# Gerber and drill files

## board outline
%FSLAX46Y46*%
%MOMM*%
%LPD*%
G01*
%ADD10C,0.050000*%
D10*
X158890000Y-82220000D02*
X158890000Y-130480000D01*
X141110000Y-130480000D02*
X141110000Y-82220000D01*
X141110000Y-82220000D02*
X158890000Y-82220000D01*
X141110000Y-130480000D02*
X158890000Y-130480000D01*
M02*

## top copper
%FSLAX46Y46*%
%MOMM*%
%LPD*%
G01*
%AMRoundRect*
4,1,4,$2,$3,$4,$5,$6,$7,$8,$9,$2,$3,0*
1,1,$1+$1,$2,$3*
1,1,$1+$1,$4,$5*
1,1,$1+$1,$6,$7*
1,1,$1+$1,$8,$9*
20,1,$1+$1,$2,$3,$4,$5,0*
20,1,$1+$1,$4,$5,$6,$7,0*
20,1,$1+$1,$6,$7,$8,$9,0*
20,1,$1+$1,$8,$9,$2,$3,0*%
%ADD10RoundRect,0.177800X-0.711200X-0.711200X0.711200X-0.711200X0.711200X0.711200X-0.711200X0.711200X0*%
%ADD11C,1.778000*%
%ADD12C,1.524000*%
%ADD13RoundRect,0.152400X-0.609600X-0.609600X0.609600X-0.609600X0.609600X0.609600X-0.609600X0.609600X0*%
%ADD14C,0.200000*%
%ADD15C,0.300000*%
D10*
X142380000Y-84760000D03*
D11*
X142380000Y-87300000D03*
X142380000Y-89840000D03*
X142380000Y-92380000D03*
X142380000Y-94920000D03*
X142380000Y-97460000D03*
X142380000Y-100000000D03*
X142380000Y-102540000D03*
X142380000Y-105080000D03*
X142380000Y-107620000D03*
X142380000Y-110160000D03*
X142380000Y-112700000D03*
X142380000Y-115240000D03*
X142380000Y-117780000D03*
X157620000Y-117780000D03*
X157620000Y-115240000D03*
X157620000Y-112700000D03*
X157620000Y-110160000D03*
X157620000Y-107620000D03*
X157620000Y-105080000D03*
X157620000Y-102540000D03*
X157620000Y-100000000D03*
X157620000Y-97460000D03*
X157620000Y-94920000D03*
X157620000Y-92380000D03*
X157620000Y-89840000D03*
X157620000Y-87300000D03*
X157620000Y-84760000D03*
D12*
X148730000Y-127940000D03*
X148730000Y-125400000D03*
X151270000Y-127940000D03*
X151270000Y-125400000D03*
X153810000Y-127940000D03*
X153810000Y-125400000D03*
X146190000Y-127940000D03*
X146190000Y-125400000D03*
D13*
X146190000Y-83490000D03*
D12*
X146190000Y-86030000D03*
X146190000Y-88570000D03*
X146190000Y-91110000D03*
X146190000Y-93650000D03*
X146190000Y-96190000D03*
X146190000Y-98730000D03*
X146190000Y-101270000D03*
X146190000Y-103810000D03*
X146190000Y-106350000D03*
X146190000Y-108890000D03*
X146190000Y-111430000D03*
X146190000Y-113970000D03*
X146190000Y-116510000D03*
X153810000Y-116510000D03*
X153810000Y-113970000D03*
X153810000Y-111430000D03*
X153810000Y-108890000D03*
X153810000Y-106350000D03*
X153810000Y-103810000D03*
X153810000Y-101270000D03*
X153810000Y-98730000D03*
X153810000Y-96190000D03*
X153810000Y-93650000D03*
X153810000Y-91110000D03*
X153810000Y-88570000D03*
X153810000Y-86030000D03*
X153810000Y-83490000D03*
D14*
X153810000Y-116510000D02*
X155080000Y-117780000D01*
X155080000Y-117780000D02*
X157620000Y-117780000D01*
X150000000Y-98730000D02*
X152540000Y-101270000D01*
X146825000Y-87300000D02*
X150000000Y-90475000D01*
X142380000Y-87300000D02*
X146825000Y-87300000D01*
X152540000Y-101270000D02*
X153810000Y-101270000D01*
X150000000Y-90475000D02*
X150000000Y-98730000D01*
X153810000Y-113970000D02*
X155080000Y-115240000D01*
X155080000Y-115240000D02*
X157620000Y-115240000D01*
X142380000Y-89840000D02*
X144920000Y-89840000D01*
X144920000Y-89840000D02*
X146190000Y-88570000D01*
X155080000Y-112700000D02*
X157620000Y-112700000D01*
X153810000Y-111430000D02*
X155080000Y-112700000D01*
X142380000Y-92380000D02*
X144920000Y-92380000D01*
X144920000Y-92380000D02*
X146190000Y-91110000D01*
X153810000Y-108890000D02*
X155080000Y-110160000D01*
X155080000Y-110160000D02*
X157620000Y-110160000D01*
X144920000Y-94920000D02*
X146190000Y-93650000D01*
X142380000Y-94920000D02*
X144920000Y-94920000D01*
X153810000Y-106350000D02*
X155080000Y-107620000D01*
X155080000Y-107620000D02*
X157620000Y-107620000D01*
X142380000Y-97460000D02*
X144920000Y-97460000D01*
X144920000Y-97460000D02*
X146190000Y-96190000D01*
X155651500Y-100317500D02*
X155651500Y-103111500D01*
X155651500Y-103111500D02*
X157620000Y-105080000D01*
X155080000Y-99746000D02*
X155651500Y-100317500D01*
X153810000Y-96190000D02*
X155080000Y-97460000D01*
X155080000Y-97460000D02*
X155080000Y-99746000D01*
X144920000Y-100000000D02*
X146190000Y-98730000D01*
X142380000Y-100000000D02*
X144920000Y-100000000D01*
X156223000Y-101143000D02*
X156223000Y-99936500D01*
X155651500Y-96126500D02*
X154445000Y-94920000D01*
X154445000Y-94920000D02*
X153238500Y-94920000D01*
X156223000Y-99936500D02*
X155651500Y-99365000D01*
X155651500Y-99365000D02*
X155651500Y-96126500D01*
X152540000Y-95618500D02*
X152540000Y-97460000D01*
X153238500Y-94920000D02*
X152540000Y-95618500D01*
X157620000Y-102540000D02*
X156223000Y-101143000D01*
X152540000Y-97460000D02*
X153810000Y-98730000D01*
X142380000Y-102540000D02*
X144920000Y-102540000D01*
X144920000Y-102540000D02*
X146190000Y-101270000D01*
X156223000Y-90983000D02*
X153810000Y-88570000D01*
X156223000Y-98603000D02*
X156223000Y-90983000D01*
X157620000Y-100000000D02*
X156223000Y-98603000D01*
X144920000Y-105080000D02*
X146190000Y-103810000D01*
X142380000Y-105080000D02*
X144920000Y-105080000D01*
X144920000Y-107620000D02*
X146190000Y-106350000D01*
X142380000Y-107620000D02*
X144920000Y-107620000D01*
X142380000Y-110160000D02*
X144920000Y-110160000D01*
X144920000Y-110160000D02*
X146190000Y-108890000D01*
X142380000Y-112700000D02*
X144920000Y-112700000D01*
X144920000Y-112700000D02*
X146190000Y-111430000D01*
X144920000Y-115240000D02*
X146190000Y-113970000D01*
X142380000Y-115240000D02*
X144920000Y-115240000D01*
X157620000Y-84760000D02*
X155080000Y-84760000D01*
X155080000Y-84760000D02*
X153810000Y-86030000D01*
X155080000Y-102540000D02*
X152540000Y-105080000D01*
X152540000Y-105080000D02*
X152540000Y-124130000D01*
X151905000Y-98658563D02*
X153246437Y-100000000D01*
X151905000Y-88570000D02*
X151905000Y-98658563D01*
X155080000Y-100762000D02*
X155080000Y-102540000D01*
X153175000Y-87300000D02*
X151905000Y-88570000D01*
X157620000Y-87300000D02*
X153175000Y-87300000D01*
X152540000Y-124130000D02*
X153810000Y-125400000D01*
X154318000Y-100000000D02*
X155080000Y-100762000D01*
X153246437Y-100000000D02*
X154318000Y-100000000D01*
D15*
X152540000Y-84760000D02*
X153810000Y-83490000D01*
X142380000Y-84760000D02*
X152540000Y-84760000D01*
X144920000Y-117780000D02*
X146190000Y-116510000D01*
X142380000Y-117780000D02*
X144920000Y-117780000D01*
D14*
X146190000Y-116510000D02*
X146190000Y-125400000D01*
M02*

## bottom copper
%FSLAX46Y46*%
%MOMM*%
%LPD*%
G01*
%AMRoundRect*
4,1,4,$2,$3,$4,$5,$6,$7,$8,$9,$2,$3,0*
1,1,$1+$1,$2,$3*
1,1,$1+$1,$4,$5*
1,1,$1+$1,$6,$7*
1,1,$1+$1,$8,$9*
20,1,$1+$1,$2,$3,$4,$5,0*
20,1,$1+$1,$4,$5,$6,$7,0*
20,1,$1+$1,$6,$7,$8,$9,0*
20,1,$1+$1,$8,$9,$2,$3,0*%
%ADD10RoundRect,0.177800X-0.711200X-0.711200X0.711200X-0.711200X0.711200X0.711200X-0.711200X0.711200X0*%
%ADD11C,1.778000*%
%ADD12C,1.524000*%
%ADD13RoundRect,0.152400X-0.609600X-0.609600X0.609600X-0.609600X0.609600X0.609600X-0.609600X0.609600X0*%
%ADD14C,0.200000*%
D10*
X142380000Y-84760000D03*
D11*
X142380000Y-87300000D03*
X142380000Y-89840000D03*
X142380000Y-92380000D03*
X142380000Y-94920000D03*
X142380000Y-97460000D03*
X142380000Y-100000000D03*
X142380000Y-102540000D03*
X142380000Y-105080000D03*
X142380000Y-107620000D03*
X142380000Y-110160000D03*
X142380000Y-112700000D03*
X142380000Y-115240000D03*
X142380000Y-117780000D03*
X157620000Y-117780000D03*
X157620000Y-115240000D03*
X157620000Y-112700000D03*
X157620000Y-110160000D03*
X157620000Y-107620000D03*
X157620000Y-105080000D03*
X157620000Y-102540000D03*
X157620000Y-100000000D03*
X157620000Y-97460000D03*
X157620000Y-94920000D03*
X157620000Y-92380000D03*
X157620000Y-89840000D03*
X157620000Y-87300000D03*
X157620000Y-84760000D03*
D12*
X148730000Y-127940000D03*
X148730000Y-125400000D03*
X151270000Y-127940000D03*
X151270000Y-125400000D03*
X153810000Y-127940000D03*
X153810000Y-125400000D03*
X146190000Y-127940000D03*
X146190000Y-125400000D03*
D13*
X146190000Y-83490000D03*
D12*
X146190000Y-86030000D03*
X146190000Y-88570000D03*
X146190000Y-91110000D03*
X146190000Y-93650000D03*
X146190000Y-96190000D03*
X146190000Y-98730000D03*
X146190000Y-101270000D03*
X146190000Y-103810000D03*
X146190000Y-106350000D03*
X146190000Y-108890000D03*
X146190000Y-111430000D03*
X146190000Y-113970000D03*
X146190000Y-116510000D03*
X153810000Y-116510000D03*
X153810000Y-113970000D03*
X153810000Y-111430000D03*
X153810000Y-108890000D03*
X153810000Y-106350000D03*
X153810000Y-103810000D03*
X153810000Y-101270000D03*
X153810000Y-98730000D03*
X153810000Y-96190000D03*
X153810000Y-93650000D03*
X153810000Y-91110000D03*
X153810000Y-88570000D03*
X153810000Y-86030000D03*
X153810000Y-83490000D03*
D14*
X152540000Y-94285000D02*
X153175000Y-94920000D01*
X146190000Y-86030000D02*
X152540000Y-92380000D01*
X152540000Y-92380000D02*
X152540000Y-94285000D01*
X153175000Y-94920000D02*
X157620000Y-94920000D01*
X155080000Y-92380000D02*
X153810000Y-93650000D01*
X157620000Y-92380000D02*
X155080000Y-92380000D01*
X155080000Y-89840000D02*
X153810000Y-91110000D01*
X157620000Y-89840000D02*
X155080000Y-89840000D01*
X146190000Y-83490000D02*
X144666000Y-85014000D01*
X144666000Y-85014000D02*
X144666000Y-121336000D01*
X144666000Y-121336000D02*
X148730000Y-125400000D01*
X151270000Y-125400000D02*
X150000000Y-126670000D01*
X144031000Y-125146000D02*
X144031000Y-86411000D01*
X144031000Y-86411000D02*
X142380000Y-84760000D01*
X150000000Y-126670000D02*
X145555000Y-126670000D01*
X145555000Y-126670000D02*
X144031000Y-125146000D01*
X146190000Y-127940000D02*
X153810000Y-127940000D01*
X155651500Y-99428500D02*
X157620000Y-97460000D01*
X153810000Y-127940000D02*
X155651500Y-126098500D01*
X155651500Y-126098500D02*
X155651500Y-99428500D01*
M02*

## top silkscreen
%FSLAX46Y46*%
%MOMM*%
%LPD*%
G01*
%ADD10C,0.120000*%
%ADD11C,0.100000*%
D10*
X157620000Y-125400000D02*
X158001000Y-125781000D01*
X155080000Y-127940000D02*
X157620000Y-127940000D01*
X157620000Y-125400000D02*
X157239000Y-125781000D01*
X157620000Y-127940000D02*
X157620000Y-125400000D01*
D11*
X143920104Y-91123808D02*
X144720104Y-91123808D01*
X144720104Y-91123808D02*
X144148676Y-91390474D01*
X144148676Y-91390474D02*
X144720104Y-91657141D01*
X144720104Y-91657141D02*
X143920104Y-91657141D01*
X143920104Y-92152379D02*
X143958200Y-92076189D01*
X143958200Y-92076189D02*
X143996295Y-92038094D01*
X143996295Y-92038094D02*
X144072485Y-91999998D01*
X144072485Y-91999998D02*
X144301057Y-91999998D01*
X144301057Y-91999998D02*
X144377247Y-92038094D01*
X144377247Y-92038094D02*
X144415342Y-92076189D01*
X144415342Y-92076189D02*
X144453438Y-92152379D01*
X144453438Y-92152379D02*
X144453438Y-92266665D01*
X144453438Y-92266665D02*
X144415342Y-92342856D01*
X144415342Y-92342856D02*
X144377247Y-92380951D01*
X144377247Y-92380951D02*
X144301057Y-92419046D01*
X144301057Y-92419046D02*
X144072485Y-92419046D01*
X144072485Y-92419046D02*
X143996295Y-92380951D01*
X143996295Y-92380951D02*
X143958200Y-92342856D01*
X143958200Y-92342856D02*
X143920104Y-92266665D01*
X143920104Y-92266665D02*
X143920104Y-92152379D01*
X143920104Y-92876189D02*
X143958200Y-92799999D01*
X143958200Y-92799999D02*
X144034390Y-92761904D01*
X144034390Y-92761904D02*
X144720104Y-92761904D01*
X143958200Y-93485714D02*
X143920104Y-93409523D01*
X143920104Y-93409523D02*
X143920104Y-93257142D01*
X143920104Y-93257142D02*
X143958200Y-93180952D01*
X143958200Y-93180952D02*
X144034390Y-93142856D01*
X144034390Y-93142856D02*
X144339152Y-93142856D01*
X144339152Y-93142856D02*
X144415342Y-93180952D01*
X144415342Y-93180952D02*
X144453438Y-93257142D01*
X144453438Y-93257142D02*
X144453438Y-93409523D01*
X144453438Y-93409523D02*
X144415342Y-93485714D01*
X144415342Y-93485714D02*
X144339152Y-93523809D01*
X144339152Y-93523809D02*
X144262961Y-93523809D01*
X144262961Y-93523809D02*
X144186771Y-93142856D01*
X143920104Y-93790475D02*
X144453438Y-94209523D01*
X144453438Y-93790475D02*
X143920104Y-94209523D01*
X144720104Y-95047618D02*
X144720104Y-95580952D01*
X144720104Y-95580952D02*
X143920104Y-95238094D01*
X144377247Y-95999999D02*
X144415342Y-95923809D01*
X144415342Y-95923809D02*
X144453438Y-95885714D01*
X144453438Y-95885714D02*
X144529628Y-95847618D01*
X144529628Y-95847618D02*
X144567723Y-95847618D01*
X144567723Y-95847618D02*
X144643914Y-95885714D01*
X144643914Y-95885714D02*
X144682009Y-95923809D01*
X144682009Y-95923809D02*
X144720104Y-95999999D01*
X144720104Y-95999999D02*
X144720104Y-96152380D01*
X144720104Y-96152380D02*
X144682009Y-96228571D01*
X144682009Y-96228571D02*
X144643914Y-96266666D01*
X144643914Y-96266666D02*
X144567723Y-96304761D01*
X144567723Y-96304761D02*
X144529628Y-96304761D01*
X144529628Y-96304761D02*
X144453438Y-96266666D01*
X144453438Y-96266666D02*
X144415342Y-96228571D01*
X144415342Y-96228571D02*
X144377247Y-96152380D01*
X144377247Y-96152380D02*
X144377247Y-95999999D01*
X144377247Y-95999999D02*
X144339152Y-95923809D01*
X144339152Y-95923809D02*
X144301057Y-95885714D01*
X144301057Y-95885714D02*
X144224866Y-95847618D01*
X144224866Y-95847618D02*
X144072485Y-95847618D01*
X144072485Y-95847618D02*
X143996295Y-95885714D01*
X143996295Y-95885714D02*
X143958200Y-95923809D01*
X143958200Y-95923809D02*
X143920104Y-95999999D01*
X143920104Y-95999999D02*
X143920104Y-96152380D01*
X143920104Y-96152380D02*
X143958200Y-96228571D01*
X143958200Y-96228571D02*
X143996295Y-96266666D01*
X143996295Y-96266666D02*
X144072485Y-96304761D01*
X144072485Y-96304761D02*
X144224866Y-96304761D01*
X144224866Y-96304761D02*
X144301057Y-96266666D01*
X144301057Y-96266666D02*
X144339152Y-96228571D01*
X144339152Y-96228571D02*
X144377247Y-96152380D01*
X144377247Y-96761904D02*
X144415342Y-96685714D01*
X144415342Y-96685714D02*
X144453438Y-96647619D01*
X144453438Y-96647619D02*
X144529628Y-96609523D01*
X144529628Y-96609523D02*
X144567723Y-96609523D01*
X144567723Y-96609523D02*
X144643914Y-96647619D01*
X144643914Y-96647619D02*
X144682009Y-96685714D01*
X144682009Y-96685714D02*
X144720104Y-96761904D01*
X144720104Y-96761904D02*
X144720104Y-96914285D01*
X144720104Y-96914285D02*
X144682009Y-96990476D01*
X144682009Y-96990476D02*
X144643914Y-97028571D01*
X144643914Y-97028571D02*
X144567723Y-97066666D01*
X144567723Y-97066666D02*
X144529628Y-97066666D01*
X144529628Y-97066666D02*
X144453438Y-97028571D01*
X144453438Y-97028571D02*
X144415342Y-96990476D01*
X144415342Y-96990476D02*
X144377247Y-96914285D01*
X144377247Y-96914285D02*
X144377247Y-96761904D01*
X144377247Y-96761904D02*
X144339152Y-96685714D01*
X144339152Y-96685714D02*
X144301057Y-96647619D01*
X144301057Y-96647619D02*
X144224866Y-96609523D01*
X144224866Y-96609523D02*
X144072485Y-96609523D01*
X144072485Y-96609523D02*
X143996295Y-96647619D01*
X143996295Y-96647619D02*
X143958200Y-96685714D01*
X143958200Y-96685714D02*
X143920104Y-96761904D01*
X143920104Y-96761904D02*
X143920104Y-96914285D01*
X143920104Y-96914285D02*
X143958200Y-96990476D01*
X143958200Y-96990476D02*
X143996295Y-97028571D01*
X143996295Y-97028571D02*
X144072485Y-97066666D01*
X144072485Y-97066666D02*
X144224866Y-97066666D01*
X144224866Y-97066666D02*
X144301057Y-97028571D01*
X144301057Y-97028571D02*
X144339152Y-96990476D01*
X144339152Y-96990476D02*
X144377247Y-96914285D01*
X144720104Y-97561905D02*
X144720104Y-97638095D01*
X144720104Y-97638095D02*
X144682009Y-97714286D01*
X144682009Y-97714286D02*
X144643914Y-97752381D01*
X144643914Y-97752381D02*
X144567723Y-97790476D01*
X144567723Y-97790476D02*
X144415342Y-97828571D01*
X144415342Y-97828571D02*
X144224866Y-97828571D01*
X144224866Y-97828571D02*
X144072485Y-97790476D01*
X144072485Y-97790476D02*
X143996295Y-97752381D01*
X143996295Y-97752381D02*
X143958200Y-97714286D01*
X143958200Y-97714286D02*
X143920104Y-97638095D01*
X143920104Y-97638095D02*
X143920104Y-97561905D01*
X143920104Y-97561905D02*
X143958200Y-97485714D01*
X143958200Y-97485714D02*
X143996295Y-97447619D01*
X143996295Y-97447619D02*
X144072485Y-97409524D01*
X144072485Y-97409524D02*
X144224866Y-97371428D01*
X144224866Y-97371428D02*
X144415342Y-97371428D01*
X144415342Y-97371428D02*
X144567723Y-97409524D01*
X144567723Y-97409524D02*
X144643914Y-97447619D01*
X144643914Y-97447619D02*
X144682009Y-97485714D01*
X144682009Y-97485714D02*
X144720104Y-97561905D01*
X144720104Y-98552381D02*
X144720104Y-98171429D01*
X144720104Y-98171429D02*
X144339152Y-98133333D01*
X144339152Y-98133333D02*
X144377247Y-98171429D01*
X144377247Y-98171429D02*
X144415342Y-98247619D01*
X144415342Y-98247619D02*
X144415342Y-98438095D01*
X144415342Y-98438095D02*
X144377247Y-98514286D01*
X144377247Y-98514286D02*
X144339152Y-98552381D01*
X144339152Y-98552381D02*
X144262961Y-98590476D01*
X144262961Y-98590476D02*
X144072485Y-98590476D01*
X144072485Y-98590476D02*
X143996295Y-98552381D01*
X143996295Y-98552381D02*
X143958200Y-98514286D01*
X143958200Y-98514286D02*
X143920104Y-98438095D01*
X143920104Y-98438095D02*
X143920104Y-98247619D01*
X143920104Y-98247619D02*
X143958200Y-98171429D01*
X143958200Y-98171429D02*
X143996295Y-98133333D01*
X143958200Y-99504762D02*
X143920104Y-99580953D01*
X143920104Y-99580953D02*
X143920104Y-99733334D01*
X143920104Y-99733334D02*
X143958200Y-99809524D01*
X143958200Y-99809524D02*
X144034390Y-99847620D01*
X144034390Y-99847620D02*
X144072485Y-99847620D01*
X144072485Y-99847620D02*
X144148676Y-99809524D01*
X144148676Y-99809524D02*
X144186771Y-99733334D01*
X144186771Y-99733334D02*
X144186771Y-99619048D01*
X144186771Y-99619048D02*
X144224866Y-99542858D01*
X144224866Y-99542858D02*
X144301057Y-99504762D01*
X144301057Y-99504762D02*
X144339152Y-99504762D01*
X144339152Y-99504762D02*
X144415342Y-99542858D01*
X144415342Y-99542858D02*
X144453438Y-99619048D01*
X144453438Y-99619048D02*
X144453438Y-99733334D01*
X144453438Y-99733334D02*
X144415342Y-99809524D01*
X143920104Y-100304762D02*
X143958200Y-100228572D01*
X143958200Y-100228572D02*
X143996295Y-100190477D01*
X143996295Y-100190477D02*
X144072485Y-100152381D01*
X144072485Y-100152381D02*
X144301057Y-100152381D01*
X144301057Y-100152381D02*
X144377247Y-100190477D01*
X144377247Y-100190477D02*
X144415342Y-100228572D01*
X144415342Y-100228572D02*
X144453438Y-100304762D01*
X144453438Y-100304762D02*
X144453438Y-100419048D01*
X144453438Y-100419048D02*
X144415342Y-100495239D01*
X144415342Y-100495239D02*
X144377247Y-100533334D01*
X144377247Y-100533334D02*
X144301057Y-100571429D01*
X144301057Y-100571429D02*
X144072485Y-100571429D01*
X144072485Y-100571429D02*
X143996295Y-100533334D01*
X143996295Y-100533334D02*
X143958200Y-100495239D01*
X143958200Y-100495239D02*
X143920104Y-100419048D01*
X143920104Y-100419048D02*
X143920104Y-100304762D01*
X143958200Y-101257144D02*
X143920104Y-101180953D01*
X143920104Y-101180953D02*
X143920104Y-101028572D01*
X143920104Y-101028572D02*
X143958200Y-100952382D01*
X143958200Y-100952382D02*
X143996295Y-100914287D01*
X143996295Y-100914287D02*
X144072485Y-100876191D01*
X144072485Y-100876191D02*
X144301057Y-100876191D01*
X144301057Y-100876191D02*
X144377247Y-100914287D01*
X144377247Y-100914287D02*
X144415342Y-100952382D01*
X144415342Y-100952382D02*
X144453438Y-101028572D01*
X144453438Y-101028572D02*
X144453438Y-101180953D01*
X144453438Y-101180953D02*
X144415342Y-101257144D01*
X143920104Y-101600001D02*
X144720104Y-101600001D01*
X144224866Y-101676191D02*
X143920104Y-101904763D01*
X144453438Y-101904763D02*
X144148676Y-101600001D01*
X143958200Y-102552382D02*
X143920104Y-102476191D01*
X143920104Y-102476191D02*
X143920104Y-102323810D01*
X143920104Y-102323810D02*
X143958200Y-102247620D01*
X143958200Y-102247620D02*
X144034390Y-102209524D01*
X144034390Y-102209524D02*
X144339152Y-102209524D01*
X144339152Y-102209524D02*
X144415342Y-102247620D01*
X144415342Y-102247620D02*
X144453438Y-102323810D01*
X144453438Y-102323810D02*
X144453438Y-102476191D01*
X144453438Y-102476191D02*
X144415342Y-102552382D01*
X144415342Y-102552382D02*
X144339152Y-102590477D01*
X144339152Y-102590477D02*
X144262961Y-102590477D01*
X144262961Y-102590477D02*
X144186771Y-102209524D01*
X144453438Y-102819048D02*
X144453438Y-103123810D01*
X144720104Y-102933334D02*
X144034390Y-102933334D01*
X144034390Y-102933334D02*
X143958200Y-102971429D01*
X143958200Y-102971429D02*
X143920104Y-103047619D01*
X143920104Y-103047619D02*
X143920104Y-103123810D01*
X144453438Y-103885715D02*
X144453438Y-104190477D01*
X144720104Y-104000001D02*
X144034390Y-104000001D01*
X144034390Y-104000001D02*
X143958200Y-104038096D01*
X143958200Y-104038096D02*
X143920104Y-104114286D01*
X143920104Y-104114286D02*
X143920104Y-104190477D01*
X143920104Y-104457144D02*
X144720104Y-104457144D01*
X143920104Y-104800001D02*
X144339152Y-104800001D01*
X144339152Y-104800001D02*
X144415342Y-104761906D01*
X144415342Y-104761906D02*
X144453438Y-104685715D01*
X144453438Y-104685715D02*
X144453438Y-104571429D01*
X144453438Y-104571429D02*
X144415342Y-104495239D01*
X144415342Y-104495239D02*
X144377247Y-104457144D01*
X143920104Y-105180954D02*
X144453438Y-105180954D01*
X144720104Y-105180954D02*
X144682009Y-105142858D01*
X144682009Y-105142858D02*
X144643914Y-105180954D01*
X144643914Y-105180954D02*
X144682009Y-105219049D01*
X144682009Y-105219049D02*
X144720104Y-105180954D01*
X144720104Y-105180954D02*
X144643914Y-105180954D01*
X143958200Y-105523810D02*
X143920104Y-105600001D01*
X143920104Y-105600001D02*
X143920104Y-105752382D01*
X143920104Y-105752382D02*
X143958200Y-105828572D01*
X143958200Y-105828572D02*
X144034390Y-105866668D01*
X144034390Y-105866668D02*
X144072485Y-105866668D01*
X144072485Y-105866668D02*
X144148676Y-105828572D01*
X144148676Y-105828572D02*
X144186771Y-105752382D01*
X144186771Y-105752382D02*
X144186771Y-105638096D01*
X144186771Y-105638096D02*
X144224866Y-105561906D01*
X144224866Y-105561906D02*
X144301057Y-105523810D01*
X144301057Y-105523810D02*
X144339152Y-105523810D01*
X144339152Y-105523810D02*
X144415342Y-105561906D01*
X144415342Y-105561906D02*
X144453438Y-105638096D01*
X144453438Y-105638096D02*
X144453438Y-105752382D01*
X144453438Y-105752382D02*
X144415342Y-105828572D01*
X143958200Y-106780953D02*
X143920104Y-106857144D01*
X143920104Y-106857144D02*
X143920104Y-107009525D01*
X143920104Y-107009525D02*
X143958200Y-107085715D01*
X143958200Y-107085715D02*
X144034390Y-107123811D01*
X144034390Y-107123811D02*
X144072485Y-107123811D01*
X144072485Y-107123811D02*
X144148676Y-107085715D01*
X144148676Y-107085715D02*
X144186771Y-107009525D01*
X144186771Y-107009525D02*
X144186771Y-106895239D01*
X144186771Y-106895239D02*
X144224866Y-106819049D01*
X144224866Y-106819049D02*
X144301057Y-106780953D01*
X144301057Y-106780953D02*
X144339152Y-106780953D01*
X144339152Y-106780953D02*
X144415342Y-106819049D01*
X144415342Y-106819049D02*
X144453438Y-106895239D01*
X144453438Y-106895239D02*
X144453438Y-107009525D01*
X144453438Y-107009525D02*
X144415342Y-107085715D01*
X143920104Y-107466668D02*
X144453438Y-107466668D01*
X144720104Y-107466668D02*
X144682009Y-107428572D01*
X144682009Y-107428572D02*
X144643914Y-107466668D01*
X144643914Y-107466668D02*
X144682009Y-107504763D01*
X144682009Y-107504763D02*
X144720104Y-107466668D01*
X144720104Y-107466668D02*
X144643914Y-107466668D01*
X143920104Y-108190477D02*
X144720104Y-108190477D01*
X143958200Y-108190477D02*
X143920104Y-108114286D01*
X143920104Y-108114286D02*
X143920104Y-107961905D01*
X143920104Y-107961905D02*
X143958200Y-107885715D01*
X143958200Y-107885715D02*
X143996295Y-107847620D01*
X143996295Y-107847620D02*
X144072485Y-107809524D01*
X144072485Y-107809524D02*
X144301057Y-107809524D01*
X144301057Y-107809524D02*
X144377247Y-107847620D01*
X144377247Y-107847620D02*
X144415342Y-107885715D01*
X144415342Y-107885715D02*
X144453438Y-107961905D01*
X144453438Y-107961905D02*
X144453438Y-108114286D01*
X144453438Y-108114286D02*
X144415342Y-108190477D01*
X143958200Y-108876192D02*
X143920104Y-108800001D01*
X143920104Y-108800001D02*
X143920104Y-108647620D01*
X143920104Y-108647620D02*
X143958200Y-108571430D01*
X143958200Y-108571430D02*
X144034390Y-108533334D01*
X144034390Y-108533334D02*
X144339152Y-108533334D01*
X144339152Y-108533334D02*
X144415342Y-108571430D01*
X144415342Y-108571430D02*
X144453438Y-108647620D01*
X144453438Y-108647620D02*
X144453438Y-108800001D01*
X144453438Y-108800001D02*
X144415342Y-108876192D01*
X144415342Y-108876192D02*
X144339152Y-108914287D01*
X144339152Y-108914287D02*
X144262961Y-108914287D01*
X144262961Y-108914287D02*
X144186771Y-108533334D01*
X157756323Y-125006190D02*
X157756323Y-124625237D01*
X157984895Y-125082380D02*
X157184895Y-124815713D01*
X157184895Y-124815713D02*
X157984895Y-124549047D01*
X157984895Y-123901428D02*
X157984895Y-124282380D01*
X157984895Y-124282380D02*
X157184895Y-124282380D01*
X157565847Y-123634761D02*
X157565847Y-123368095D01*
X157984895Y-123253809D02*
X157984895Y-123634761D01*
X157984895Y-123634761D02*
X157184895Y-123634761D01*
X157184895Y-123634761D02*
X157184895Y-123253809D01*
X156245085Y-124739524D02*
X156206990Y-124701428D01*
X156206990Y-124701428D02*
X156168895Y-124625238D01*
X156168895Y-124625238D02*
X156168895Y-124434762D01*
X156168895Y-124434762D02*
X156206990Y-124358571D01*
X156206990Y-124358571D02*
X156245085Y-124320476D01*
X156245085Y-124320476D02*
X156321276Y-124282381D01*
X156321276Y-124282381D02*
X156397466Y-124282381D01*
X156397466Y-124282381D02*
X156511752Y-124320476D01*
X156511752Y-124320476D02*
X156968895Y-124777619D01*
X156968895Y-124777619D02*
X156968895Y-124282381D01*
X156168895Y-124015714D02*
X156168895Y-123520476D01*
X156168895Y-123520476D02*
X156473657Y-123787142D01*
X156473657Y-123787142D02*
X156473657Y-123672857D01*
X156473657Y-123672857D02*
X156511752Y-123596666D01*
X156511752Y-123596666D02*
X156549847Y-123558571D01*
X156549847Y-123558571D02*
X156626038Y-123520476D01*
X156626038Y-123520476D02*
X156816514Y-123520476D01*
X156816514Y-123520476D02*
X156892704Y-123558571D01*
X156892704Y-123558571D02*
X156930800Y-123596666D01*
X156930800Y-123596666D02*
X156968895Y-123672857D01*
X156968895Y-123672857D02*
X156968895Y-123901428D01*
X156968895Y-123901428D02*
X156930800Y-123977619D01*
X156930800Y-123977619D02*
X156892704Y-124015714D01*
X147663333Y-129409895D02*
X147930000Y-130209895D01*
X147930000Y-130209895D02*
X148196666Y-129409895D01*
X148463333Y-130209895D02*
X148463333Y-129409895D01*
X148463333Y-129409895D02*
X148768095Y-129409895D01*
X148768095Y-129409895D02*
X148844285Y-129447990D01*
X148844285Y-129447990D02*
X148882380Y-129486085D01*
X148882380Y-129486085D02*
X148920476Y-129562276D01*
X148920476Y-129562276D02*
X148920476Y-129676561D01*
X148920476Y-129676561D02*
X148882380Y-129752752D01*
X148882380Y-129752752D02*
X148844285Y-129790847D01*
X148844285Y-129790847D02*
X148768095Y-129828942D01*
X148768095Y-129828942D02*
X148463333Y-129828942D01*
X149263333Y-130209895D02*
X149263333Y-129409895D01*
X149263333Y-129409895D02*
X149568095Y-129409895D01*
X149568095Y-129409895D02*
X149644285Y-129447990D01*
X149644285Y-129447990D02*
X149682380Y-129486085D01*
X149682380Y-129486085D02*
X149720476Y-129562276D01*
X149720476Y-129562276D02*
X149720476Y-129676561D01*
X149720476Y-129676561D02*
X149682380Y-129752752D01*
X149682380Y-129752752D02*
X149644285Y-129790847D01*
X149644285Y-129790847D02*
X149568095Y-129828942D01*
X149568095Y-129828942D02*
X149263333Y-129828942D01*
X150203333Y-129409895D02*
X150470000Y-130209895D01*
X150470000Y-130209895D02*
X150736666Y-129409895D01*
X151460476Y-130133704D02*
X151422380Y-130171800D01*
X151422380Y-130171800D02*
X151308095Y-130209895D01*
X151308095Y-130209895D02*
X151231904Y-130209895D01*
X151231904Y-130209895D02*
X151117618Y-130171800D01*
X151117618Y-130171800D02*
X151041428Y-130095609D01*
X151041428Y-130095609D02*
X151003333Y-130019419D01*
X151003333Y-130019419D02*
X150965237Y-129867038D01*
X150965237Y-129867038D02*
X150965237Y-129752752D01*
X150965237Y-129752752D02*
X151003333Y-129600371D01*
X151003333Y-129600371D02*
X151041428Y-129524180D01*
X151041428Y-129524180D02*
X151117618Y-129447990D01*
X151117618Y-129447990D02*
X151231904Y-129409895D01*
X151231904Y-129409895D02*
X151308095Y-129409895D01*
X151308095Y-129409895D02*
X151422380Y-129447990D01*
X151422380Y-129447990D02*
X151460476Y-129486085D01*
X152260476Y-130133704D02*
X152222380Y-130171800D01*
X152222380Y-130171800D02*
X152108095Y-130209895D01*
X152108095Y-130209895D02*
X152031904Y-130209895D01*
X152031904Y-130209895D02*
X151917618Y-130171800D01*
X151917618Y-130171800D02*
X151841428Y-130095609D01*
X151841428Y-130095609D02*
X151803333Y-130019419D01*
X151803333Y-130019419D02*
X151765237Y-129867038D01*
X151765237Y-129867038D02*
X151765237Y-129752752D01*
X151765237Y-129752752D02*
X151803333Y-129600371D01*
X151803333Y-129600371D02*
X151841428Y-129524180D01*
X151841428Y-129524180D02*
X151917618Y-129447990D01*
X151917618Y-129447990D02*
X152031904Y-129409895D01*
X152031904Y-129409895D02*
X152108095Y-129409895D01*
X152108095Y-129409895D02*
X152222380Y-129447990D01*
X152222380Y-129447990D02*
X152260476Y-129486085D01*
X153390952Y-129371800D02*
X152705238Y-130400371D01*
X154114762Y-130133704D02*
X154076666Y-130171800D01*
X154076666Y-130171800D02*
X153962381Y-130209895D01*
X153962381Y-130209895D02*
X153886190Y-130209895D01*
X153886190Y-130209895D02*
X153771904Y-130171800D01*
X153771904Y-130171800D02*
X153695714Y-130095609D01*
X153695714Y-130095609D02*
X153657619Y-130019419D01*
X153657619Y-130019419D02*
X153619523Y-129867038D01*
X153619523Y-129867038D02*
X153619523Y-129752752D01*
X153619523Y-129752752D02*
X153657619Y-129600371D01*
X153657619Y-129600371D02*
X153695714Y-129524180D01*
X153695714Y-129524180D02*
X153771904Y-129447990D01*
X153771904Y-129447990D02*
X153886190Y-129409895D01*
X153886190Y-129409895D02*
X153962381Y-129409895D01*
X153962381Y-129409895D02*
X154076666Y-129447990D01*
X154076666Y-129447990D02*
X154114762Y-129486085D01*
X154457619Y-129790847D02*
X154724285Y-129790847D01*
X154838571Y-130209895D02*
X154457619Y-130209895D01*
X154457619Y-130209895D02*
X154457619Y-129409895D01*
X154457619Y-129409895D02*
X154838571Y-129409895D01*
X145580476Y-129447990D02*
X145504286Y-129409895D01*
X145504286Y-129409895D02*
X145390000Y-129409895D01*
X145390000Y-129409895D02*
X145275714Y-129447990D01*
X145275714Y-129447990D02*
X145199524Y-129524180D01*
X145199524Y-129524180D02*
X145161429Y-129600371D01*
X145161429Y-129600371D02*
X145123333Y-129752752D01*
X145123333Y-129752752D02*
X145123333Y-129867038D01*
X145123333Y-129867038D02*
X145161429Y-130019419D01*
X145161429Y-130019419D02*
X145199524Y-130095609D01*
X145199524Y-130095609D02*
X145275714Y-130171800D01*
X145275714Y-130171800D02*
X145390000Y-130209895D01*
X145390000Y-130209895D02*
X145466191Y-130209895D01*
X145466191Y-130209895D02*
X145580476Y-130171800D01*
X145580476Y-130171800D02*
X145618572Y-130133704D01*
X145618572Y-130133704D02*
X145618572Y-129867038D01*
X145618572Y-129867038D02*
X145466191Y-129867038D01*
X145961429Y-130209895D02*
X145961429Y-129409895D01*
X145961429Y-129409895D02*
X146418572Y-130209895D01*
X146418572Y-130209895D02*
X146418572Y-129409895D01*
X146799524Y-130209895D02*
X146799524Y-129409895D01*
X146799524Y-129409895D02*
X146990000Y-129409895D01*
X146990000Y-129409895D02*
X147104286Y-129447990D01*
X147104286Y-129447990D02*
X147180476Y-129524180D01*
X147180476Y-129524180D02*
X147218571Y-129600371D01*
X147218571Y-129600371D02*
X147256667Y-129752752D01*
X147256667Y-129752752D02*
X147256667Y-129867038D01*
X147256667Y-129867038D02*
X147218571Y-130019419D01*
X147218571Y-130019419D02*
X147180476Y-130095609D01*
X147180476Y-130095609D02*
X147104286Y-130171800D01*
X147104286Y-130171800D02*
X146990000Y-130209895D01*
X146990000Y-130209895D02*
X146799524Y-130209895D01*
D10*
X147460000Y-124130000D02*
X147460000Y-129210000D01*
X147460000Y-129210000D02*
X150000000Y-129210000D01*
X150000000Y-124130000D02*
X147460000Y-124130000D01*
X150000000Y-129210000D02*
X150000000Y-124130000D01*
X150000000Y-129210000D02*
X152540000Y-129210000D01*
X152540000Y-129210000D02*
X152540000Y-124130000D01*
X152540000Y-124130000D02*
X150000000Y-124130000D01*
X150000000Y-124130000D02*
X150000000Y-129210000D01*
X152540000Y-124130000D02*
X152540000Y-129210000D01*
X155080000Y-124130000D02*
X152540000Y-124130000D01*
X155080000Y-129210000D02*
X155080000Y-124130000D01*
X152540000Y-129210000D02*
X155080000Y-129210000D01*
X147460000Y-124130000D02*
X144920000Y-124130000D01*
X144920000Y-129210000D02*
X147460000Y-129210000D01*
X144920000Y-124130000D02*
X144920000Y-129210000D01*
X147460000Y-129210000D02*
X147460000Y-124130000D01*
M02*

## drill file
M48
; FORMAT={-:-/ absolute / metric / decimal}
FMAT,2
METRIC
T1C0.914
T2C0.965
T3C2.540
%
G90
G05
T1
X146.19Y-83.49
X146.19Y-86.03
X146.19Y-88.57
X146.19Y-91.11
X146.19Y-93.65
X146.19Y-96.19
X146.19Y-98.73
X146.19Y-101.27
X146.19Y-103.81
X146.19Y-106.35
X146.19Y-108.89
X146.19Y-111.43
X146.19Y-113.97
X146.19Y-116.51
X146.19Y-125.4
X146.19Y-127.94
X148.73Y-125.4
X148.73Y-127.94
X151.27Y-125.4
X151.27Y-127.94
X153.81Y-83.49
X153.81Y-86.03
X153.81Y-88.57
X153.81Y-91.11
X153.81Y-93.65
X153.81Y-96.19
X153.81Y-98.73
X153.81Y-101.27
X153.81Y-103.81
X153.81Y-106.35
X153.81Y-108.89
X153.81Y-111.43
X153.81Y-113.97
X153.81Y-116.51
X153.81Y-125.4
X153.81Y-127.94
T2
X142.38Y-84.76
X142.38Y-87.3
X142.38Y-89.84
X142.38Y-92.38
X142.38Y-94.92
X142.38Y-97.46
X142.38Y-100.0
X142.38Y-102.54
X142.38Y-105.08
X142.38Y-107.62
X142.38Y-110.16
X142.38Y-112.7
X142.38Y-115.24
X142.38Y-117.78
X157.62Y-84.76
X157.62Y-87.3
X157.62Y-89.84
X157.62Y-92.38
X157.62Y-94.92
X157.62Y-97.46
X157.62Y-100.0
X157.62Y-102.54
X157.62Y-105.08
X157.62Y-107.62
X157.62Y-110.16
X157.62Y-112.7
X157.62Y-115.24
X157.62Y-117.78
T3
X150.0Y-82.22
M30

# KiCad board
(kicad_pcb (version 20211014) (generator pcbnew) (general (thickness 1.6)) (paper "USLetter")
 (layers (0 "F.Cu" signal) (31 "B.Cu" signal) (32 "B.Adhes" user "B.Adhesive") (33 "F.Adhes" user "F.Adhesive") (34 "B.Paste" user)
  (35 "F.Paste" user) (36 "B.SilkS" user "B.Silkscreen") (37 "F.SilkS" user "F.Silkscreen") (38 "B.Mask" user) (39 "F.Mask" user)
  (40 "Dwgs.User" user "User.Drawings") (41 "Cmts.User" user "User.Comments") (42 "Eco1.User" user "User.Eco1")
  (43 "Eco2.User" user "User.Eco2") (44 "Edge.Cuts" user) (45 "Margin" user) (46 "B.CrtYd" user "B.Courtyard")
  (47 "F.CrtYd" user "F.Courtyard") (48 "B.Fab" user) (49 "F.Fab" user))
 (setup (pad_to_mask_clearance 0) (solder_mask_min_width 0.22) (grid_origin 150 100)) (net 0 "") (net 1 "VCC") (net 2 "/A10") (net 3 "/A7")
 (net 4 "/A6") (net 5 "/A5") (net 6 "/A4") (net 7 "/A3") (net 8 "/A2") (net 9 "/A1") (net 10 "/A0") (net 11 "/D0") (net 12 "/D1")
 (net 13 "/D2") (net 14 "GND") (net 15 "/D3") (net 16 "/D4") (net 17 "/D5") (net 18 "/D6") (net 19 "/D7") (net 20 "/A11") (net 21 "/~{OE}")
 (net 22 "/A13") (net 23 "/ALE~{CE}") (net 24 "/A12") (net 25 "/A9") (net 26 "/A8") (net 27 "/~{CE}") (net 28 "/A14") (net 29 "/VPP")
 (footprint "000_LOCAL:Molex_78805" (layer "F.Cu") (at 150 101.27)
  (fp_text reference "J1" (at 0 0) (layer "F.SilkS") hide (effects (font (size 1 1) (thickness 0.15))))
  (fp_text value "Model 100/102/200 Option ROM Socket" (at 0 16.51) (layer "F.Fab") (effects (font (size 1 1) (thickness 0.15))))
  (pad "1" thru_hole roundrect locked (at -7.62 -16.51) (size 1.778 1.778) (drill 0.9652) (layers *.Cu *.Mask) (roundrect_rratio 0.1)
   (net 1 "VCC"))
  (pad "2" thru_hole circle locked (at -7.62 -13.97) (size 1.778 1.778) (drill 0.9652) (layers *.Cu *.Mask) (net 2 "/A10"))
  (pad "3" thru_hole circle locked (at -7.62 -11.43) (size 1.778 1.778) (drill 0.9652) (layers *.Cu *.Mask) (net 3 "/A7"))
  (pad "4" thru_hole circle locked (at -7.62 -8.89) (size 1.778 1.778) (drill 0.9652) (layers *.Cu *.Mask) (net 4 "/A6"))
  (pad "5" thru_hole circle locked (at -7.62 -6.35) (size 1.778 1.778) (drill 0.9652) (layers *.Cu *.Mask) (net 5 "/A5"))
  (pad "6" thru_hole circle locked (at -7.62 -3.81) (size 1.778 1.778) (drill 0.9652) (layers *.Cu *.Mask) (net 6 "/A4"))
  (pad "7" thru_hole circle locked (at -7.62 -1.27) (size 1.778 1.778) (drill 0.9652) (layers *.Cu *.Mask) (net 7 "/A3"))
  (pad "8" thru_hole circle locked (at -7.62 1.27) (size 1.778 1.778) (drill 0.9652) (layers *.Cu *.Mask) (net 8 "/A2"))
  (pad "9" thru_hole circle locked (at -7.62 3.81) (size 1.778 1.778) (drill 0.9652) (layers *.Cu *.Mask) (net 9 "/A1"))
  (pad "10" thru_hole circle locked (at -7.62 6.35) (size 1.778 1.778) (drill 0.9652) (layers *.Cu *.Mask) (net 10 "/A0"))
  (pad "11" thru_hole circle locked (at -7.62 8.89) (size 1.778 1.778) (drill 0.9652) (layers *.Cu *.Mask) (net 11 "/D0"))
  (pad "12" thru_hole circle locked (at -7.62 11.43) (size 1.778 1.778) (drill 0.9652) (layers *.Cu *.Mask) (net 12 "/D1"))
  (pad "13" thru_hole circle locked (at -7.62 13.97) (size 1.778 1.778) (drill 0.9652) (layers *.Cu *.Mask) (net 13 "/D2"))
  (pad "14" thru_hole circle locked (at -7.62 16.51) (size 1.778 1.778) (drill 0.9652) (layers *.Cu *.Mask) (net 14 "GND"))
  (pad "15" thru_hole circle locked (at 7.62 16.51) (size 1.778 1.778) (drill 0.9652) (layers *.Cu *.Mask) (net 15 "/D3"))
  (pad "16" thru_hole circle locked (at 7.62 13.97) (size 1.778 1.778) (drill 0.9652) (layers *.Cu *.Mask) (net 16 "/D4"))
  (pad "17" thru_hole circle locked (at 7.62 11.43) (size 1.778 1.778) (drill 0.9652) (layers *.Cu *.Mask) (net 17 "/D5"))
  (pad "18" thru_hole circle locked (at 7.62 8.89) (size 1.778 1.778) (drill 0.9652) (layers *.Cu *.Mask) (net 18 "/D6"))
  (pad "19" thru_hole circle locked (at 7.62 6.35) (size 1.778 1.778) (drill 0.9652) (layers *.Cu *.Mask) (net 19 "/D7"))
  (pad "20" thru_hole circle locked (at 7.62 3.81) (size 1.778 1.778) (drill 0.9652) (layers *.Cu *.Mask) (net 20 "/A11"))
  (pad "21" thru_hole circle locked (at 7.62 1.27) (size 1.778 1.778) (drill 0.9652) (layers *.Cu *.Mask) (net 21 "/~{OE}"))
  (pad "22" thru_hole circle locked (at 7.62 -1.27) (size 1.778 1.778) (drill 0.9652) (layers *.Cu *.Mask) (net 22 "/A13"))
  (pad "23" thru_hole circle locked (at 7.62 -3.81) (size 1.778 1.778) (drill 0.9652) (layers *.Cu *.Mask) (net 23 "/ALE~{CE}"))
  (pad "24" thru_hole circle locked (at 7.62 -6.35) (size 1.778 1.778) (drill 0.9652) (layers *.Cu *.Mask) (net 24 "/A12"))
  (pad "25" thru_hole circle locked (at 7.62 -8.89) (size 1.778 1.778) (drill 0.9652) (layers *.Cu *.Mask) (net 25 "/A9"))
  (pad "26" thru_hole circle locked (at 7.62 -11.43) (size 1.778 1.778) (drill 0.9652) (layers *.Cu *.Mask) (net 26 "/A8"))
  (pad "27" thru_hole circle locked (at 7.62 -13.97) (size 1.778 1.778) (drill 0.9652) (layers *.Cu *.Mask) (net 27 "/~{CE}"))
  (pad "28" thru_hole circle locked (at 7.62 -16.51) (size 1.778 1.778) (drill 0.9652) (layers *.Cu *.Mask) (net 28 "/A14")))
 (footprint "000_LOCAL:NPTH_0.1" (layer "F.Cu") (at 150 82.22)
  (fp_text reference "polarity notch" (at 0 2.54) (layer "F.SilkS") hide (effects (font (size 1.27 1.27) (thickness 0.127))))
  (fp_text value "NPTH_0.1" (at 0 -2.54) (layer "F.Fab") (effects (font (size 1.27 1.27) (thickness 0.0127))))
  (pad "" np_thru_hole circle locked (at 0 0) (size 2.54 2.54) (drill 2.54) (layers *.Cu *.Mask)))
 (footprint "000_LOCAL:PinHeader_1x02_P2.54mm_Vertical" (layer "F.Cu") (at 148.73 127.94 180)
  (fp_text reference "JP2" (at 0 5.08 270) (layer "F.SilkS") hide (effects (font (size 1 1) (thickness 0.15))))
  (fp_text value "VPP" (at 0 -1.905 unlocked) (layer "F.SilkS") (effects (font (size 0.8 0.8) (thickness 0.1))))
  (fp_line (start 1.27 3.81) (end 1.27 -1.27) (layer "F.SilkS") (width 0.12))
  (fp_line (start 1.27 -1.27) (end -1.27 -1.27) (layer "F.SilkS") (width 0.12))
  (fp_line (start -1.27 3.81) (end 1.27 3.81) (layer "F.SilkS") (width 0.12))
  (fp_line (start -1.27 -1.27) (end -1.27 3.81) (layer "F.SilkS") (width 0.12))
  (pad "1" thru_hole circle locked (at 0 0 180) (size 1.524 1.524) (drill 0.9144) (layers *.Cu *.Mask) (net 23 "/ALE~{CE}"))
  (pad "2" thru_hole circle locked (at 0 2.54 180) (size 1.524 1.524) (drill 0.9144) (layers *.Cu *.Mask) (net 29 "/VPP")))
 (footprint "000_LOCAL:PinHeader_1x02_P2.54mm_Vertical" (layer "F.Cu") (at 151.27 127.94 180)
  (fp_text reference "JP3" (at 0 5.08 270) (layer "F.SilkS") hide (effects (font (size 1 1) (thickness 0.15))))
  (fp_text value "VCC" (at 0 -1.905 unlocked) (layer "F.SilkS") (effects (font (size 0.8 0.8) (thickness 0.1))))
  (fp_line (start 1.27 -1.27) (end -1.27 -1.27) (layer "F.SilkS") (width 0.12))
  (fp_line (start -1.27 -1.27) (end -1.27 3.81) (layer "F.SilkS") (width 0.12))
  (fp_line (start -1.27 3.81) (end 1.27 3.81) (layer "F.SilkS") (width 0.12))
  (fp_line (start 1.27 3.81) (end 1.27 -1.27) (layer "F.SilkS") (width 0.12))
  (pad "1" thru_hole circle locked (at 0 0 180) (size 1.524 1.524) (drill 0.9144) (layers *.Cu *.Mask) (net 23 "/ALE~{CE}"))
  (pad "2" thru_hole circle locked (at 0 2.54 180) (size 1.524 1.524) (drill 0.9144) (layers *.Cu *.Mask) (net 1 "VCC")))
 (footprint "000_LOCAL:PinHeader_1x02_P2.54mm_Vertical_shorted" (layer "F.Cu") (at 153.81 127.94 180)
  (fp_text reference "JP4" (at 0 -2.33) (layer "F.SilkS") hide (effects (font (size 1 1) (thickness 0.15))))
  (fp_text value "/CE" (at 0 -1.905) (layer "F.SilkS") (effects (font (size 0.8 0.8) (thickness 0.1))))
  (fp_line (start 1.27 3.81) (end 1.27 -1.27) (layer "F.SilkS") (width 0.12))
  (fp_line (start -1.27 3.81) (end 1.27 3.81) (layer "F.SilkS") (width 0.12))
  (fp_line (start -1.27 -1.27) (end -1.27 3.81) (layer "F.SilkS") (width 0.12))
  (fp_line (start 1.27 -1.27) (end -1.27 -1.27) (layer "F.SilkS") (width 0.12))
  (pad "1" thru_hole circle locked (at 0 0 180) (size 1.524 1.524) (drill 0.9144) (layers *.Cu *.Mask) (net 23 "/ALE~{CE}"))
  (pad "2" thru_hole circle locked (at 0 2.54 180) (size 1.524 1.524) (drill 0.9144) (layers *.Cu *.Mask) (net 27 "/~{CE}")))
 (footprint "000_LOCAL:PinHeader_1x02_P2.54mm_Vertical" (layer "F.Cu") (at 146.19 127.94 180)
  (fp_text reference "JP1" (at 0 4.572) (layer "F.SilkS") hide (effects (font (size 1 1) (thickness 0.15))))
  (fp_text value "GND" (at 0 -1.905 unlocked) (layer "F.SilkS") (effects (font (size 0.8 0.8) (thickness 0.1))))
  (fp_line (start -1.27 3.81) (end 1.27 3.81) (layer "F.SilkS") (width 0.12))
  (fp_line (start 1.27 -1.27) (end -1.27 -1.27) (layer "F.SilkS") (width 0.12))
  (fp_line (start 1.27 3.81) (end 1.27 -1.27) (layer "F.SilkS") (width 0.12))
  (fp_line (start -1.27 -1.27) (end -1.27 3.81) (layer "F.SilkS") (width 0.12))
  (pad "1" thru_hole circle locked (at 0 0 180) (size 1.524 1.524) (drill 0.9144) (layers *.Cu *.Mask) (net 23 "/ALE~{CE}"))
  (pad "2" thru_hole circle locked (at 0 2.54 180) (size 1.524 1.524) (drill 0.9144) (layers *.Cu *.Mask) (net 14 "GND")))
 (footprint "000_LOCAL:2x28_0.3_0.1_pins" (layer "F.Cu") (at 150 100)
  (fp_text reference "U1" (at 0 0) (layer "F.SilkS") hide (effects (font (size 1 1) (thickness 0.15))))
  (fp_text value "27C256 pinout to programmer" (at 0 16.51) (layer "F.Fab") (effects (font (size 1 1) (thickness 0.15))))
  (pad "1" thru_hole roundrect locked (at -3.81 -16.51) (size 1.524 1.524) (drill 0.9144) (layers *.Cu *.Mask) (roundrect_rratio 0.1)
   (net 29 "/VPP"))
  (pad "2" thru_hole circle locked (at -3.81 -13.97) (size 1.524 1.524) (drill 0.9144) (layers *.Cu *.Mask) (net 24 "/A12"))
  (pad "3" thru_hole circle locked (at -3.81 -11.43) (size 1.524 1.524) (drill 0.9144) (layers *.Cu *.Mask) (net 3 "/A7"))
  (pad "4" thru_hole circle locked (at -3.81 -8.89) (size 1.524 1.524) (drill 0.9144) (layers *.Cu *.Mask) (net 4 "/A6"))
  (pad "5" thru_hole circle locked (at -3.81 -6.35) (size 1.524 1.524) (drill 0.9144) (layers *.Cu *.Mask) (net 5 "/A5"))
  (pad "6" thru_hole circle locked (at -3.81 -3.81) (size 1.524 1.524) (drill 0.9144) (layers *.Cu *.Mask) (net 6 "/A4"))
  (pad "7" thru_hole circle locked (at -3.81 -1.27) (size 1.524 1.524) (drill 0.9144) (layers *.Cu *.Mask) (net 7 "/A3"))
  (pad "8" thru_hole circle locked (at -3.81 1.27) (size 1.524 1.524) (drill 0.9144) (layers *.Cu *.Mask) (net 8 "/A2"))
  (pad "9" thru_hole circle locked (at -3.81 3.81) (size 1.524 1.524) (drill 0.9144) (layers *.Cu *.Mask) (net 9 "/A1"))
  (pad "10" thru_hole circle locked (at -3.81 6.35) (size 1.524 1.524) (drill 0.9144) (layers *.Cu *.Mask) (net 10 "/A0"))
  (pad "11" thru_hole circle locked (at -3.81 8.89) (size 1.524 1.524) (drill 0.9144) (layers *.Cu *.Mask) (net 11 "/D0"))
  (pad "12" thru_hole circle locked (at -3.81 11.43) (size 1.524 1.524) (drill 0.9144) (layers *.Cu *.Mask) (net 12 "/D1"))
  (pad "13" thru_hole circle locked (at -3.81 13.97) (size 1.524 1.524) (drill 0.9144) (layers *.Cu *.Mask) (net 13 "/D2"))
  (pad "14" thru_hole circle locked (at -3.81 16.51) (size 1.524 1.524) (drill 0.9144) (layers *.Cu *.Mask) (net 14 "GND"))
  (pad "15" thru_hole circle locked (at 3.81 16.51) (size 1.524 1.524) (drill 0.9144) (layers *.Cu *.Mask) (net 15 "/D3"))
  (pad "16" thru_hole circle locked (at 3.81 13.97) (size 1.524 1.524) (drill 0.9144) (layers *.Cu *.Mask) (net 16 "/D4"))
  (pad "17" thru_hole circle locked (at 3.81 11.43) (size 1.524 1.524) (drill 0.9144) (layers *.Cu *.Mask) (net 17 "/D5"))
  (pad "18" thru_hole circle locked (at 3.81 8.89) (size 1.524 1.524) (drill 0.9144) (layers *.Cu *.Mask) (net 18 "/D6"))
  (pad "19" thru_hole circle locked (at 3.81 6.35) (size 1.524 1.524) (drill 0.9144) (layers *.Cu *.Mask) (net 19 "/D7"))
  (pad "20" thru_hole circle locked (at 3.81 3.81) (size 1.524 1.524) (drill 0.9144) (layers *.Cu *.Mask) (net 27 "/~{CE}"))
  (pad "21" thru_hole circle locked (at 3.81 1.27) (size 1.524 1.524) (drill 0.9144) (layers *.Cu *.Mask) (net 2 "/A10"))
  (pad "22" thru_hole circle locked (at 3.81 -1.27) (size 1.524 1.524) (drill 0.9144) (layers *.Cu *.Mask) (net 21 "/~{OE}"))
  (pad "23" thru_hole circle locked (at 3.81 -3.81) (size 1.524 1.524) (drill 0.9144) (layers *.Cu *.Mask) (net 20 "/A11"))
  (pad "24" thru_hole circle locked (at 3.81 -6.35) (size 1.524 1.524) (drill 0.9144) (layers *.Cu *.Mask) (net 25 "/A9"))
  (pad "25" thru_hole circle locked (at 3.81 -8.89) (size 1.524 1.524) (drill 0.9144) (layers *.Cu *.Mask) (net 26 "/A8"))
  (pad "26" thru_hole circle locked (at 3.81 -11.43) (size 1.524 1.524) (drill 0.9144) (layers *.Cu *.Mask) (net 22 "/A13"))
  (pad "27" thru_hole circle locked (at 3.81 -13.97) (size 1.524 1.524) (drill 0.9144) (layers *.Cu *.Mask) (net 28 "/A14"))
  (pad "28" thru_hole circle locked (at 3.81 -16.51) (size 1.524 1.524) (drill 0.9144) (layers *.Cu *.Mask) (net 1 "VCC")))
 (gr_line (start 157.62 125.4) (end 158.001 125.781) (layer "F.SilkS") (width 0.12))
 (gr_line (start 155.08 127.94) (end 157.62 127.94) (layer "F.SilkS") (width 0.12))
 (gr_line (start 157.62 125.4) (end 157.239 125.781) (layer "F.SilkS") (width 0.12))
 (gr_line (start 157.62 127.94) (end 157.62 125.4) (layer "F.SilkS") (width 0.12))
 (gr_line (start 158.89 82.22) (end 158.89 130.48) (layer "Edge.Cuts") (width 0.05))
 (gr_line (start 141.11 130.48) (end 141.11 82.22) (layer "Edge.Cuts") (width 0.05))
 (gr_line (start 141.11 82.22) (end 158.89 82.22) (layer "Edge.Cuts") (width 0.05))
 (gr_line (start 141.11 130.48) (end 158.89 130.48) (layer "Edge.Cuts") (width 0.05))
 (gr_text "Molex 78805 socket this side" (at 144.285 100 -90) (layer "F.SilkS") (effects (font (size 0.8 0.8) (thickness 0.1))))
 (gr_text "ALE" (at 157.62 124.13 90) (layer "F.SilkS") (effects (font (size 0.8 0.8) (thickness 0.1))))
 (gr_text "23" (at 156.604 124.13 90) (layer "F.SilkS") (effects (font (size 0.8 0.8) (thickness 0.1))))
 (segment (start 153.81 116.51) (end 155.08 117.78) (width 0.2) (layer "F.Cu") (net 15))
 (segment (start 155.08 117.78) (end 157.62 117.78) (width 0.2) (layer "F.Cu") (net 15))
 (segment (start 150 98.73) (end 152.54 101.27) (width 0.2) (layer "F.Cu") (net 2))
 (segment (start 146.825 87.3) (end 150 90.475) (width 0.2) (layer "F.Cu") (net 2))
 (segment (start 142.38 87.3) (end 146.825 87.3) (width 0.2) (layer "F.Cu") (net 2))
 (segment (start 152.54 101.27) (end 153.81 101.27) (width 0.2) (layer "F.Cu") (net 2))
 (segment (start 150 90.475) (end 150 98.73) (width 0.2) (layer "F.Cu") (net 2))
 (segment (start 153.81 113.97) (end 155.08 115.24) (width 0.2) (layer "F.Cu") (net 16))
 (segment (start 155.08 115.24) (end 157.62 115.24) (width 0.2) (layer "F.Cu") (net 16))
 (segment (start 142.38 89.84) (end 144.92 89.84) (width 0.2) (layer "F.Cu") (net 3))
 (segment (start 144.92 89.84) (end 146.19 88.57) (width 0.2) (layer "F.Cu") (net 3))
 (segment (start 155.08 112.7) (end 157.62 112.7) (width 0.2) (layer "F.Cu") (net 17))
 (segment (start 153.81 111.43) (end 155.08 112.7) (width 0.2) (layer "F.Cu") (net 17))
 (segment (start 142.38 92.38) (end 144.92 92.38) (width 0.2) (layer "F.Cu") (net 4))
 (segment (start 144.92 92.38) (end 146.19 91.11) (width 0.2) (layer "F.Cu") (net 4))
 (segment (start 153.81 108.89) (end 155.08 110.16) (width 0.2) (layer "F.Cu") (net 18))
 (segment (start 155.08 110.16) (end 157.62 110.16) (width 0.2) (layer "F.Cu") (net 18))
 (segment (start 144.92 94.92) (end 146.19 93.65) (width 0.2) (layer "F.Cu") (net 5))
 (segment (start 142.38 94.92) (end 144.92 94.92) (width 0.2) (layer "F.Cu") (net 5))
 (segment (start 153.81 106.35) (end 155.08 107.62) (width 0.2) (layer "F.Cu") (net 19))
 (segment (start 155.08 107.62) (end 157.62 107.62) (width 0.2) (layer "F.Cu") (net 19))
 (segment (start 142.38 97.46) (end 144.92 97.46) (width 0.2) (layer "F.Cu") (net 6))
 (segment (start 144.92 97.46) (end 146.19 96.19) (width 0.2) (layer "F.Cu") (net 6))
 (segment (start 155.6515 100.3175) (end 155.6515 103.1115) (width 0.2) (layer "F.Cu") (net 20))
 (segment (start 155.6515 103.1115) (end 157.62 105.08) (width 0.2) (layer "F.Cu") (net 20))
 (segment (start 155.08 99.746) (end 155.6515 100.3175) (width 0.2) (layer "F.Cu") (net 20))
 (segment (start 153.81 96.19) (end 155.08 97.46) (width 0.2) (layer "F.Cu") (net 20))
 (segment (start 155.08 97.46) (end 155.08 99.746) (width 0.2) (layer "F.Cu") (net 20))
 (segment (start 144.92 100) (end 146.19 98.73) (width 0.2) (layer "F.Cu") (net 7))
 (segment (start 142.38 100) (end 144.92 100) (width 0.2) (layer "F.Cu") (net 7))
 (segment (start 156.223 101.143) (end 156.223 99.9365) (width 0.2) (layer "F.Cu") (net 21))
 (segment (start 155.6515 96.1265) (end 154.445 94.92) (width 0.2) (layer "F.Cu") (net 21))
 (segment (start 154.445 94.92) (end 153.2385 94.92) (width 0.2) (layer "F.Cu") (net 21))
 (segment (start 156.223 99.9365) (end 155.6515 99.365) (width 0.2) (layer "F.Cu") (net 21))
 (segment (start 155.6515 99.365) (end 155.6515 96.1265) (width 0.2) (layer "F.Cu") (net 21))
 (segment (start 152.54 95.6185) (end 152.54 97.46) (width 0.2) (layer "F.Cu") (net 21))
 (segment (start 153.2385 94.92) (end 152.54 95.6185) (width 0.2) (layer "F.Cu") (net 21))
 (segment (start 157.62 102.54) (end 156.223 101.143) (width 0.2) (layer "F.Cu") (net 21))
 (segment (start 152.54 97.46) (end 153.81 98.73) (width 0.2) (layer "F.Cu") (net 21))
 (segment (start 142.38 102.54) (end 144.92 102.54) (width 0.2) (layer "F.Cu") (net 8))
 (segment (start 144.92 102.54) (end 146.19 101.27) (width 0.2) (layer "F.Cu") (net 8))
 (segment (start 156.223 90.983) (end 153.81 88.57) (width 0.2) (layer "F.Cu") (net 22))
 (segment (start 156.223 98.603) (end 156.223 90.983) (width 0.2) (layer "F.Cu") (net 22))
 (segment (start 157.62 100) (end 156.223 98.603) (width 0.2) (layer "F.Cu") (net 22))
 (segment (start 144.92 105.08) (end 146.19 103.81) (width 0.2) (layer "F.Cu") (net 9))
 (segment (start 142.38 105.08) (end 144.92 105.08) (width 0.2) (layer "F.Cu") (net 9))
 (segment (start 144.92 107.62) (end 146.19 106.35) (width 0.2) (layer "F.Cu") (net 10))
 (segment (start 142.38 107.62) (end 144.92 107.62) (width 0.2) (layer "F.Cu") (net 10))
 (segment (start 152.54 94.285) (end 153.175 94.92) (width 0.2) (layer "B.Cu") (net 24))
 (segment (start 146.19 86.03) (end 152.54 92.38) (width 0.2) (layer "B.Cu") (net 24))
 (segment (start 152.54 92.38) (end 152.54 94.285) (width 0.2) (layer "B.Cu") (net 24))
 (segment (start 153.175 94.92) (end 157.62 94.92) (width 0.2) (layer "B.Cu") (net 24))
 (segment (start 142.38 110.16) (end 144.92 110.16) (width 0.2) (layer "F.Cu") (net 11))
 (segment (start 144.92 110.16) (end 146.19 108.89) (width 0.2) (layer "F.Cu") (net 11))
 (segment (start 155.08 92.38) (end 153.81 93.65) (width 0.2) (layer "B.Cu") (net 25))
 (segment (start 157.62 92.38) (end 155.08 92.38) (width 0.2) (layer "B.Cu") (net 25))
 (segment (start 142.38 112.7) (end 144.92 112.7) (width 0.2) (layer "F.Cu") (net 12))
 (segment (start 144.92 112.7) (end 146.19 111.43) (width 0.2) (layer "F.Cu") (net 12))
 (segment (start 155.08 89.84) (end 153.81 91.11) (width 0.2) (layer "B.Cu") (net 26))
 (segment (start 157.62 89.84) (end 155.08 89.84) (width 0.2) (layer "B.Cu") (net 26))
 (segment (start 144.92 115.24) (end 146.19 113.97) (width 0.2) (layer "F.Cu") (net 13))
 (segment (start 142.38 115.24) (end 144.92 115.24) (width 0.2) (layer "F.Cu") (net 13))
 (segment (start 157.62 84.76) (end 155.08 84.76) (width 0.2) (layer "F.Cu") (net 28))
 (segment (start 155.08 84.76) (end 153.81 86.03) (width 0.2) (layer "F.Cu") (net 28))
 (segment (start 155.08 102.54) (end 152.54 105.08) (width 0.2) (layer "F.Cu") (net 27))
 (segment (start 152.54 105.08) (end 152.54 124.13) (width 0.2) (layer "F.Cu") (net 27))
 (segment (start 151.905 98.658563) (end 153.246437 100) (width 0.2) (layer "F.Cu") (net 27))
 (segment (start 151.905 88.57) (end 151.905 98.658563) (width 0.2) (layer "F.Cu") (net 27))
 (segment (start 155.08 100.762) (end 155.08 102.54) (width 0.2) (layer "F.Cu") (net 27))
 (segment (start 153.175 87.3) (end 151.905 88.57) (width 0.2) (layer "F.Cu") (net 27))
 (segment (start 157.62 87.3) (end 153.175 87.3) (width 0.2) (layer "F.Cu") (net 27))
 (segment (start 152.54 124.13) (end 153.81 125.4) (width 0.2) (layer "F.Cu") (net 27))
 (segment (start 154.318 100) (end 155.08 100.762) (width 0.2) (layer "F.Cu") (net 27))
 (segment (start 153.246437 100) (end 154.318 100) (width 0.2) (layer "F.Cu") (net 27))
 (segment (start 146.19 83.49) (end 144.666 85.014) (width 0.2) (layer "B.Cu") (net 29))
 (segment (start 144.666 85.014) (end 144.666 121.336) (width 0.2) (layer "B.Cu") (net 29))
 (segment (start 144.666 121.336) (end 148.73 125.4) (width 0.2) (layer "B.Cu") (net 29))
 (segment (start 152.54 84.76) (end 153.81 83.49) (width 0.3) (layer "F.Cu") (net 1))
 (segment (start 142.38 84.76) (end 152.54 84.76) (width 0.3) (layer "F.Cu") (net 1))
 (segment (start 151.27 125.4) (end 150 126.67) (width 0.2) (layer "B.Cu") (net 1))
 (segment (start 144.031 125.146) (end 144.031 86.411) (width 0.2) (layer "B.Cu") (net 1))
 (segment (start 144.031 86.411) (end 142.38 84.76) (width 0.2) (layer "B.Cu") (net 1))
 (segment (start 150 126.67) (end 145.555 126.67) (width 0.2) (layer "B.Cu") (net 1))
 (segment (start 145.555 126.67) (end 144.031 125.146) (width 0.2) (layer "B.Cu") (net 1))
 (segment (start 146.19 127.94) (end 153.81 127.94) (width 0.2) (layer "B.Cu") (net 23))
 (segment (start 155.6515 99.4285) (end 157.62 97.46) (width 0.2) (layer "B.Cu") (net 23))
 (segment (start 153.81 127.94) (end 155.6515 126.0985) (width 0.2) (layer "B.Cu") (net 23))
 (segment (start 155.6515 126.0985) (end 155.6515 99.4285) (width 0.2) (layer "B.Cu") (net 23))
 (segment (start 144.92 117.78) (end 146.19 116.51) (width 0.3) (layer "F.Cu") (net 14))
 (segment (start 142.38 117.78) (end 144.92 117.78) (width 0.3) (layer "F.Cu") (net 14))
 (segment (start 146.19 116.51) (end 146.19 125.4) (width 0.2) (layer "F.Cu") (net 14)))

